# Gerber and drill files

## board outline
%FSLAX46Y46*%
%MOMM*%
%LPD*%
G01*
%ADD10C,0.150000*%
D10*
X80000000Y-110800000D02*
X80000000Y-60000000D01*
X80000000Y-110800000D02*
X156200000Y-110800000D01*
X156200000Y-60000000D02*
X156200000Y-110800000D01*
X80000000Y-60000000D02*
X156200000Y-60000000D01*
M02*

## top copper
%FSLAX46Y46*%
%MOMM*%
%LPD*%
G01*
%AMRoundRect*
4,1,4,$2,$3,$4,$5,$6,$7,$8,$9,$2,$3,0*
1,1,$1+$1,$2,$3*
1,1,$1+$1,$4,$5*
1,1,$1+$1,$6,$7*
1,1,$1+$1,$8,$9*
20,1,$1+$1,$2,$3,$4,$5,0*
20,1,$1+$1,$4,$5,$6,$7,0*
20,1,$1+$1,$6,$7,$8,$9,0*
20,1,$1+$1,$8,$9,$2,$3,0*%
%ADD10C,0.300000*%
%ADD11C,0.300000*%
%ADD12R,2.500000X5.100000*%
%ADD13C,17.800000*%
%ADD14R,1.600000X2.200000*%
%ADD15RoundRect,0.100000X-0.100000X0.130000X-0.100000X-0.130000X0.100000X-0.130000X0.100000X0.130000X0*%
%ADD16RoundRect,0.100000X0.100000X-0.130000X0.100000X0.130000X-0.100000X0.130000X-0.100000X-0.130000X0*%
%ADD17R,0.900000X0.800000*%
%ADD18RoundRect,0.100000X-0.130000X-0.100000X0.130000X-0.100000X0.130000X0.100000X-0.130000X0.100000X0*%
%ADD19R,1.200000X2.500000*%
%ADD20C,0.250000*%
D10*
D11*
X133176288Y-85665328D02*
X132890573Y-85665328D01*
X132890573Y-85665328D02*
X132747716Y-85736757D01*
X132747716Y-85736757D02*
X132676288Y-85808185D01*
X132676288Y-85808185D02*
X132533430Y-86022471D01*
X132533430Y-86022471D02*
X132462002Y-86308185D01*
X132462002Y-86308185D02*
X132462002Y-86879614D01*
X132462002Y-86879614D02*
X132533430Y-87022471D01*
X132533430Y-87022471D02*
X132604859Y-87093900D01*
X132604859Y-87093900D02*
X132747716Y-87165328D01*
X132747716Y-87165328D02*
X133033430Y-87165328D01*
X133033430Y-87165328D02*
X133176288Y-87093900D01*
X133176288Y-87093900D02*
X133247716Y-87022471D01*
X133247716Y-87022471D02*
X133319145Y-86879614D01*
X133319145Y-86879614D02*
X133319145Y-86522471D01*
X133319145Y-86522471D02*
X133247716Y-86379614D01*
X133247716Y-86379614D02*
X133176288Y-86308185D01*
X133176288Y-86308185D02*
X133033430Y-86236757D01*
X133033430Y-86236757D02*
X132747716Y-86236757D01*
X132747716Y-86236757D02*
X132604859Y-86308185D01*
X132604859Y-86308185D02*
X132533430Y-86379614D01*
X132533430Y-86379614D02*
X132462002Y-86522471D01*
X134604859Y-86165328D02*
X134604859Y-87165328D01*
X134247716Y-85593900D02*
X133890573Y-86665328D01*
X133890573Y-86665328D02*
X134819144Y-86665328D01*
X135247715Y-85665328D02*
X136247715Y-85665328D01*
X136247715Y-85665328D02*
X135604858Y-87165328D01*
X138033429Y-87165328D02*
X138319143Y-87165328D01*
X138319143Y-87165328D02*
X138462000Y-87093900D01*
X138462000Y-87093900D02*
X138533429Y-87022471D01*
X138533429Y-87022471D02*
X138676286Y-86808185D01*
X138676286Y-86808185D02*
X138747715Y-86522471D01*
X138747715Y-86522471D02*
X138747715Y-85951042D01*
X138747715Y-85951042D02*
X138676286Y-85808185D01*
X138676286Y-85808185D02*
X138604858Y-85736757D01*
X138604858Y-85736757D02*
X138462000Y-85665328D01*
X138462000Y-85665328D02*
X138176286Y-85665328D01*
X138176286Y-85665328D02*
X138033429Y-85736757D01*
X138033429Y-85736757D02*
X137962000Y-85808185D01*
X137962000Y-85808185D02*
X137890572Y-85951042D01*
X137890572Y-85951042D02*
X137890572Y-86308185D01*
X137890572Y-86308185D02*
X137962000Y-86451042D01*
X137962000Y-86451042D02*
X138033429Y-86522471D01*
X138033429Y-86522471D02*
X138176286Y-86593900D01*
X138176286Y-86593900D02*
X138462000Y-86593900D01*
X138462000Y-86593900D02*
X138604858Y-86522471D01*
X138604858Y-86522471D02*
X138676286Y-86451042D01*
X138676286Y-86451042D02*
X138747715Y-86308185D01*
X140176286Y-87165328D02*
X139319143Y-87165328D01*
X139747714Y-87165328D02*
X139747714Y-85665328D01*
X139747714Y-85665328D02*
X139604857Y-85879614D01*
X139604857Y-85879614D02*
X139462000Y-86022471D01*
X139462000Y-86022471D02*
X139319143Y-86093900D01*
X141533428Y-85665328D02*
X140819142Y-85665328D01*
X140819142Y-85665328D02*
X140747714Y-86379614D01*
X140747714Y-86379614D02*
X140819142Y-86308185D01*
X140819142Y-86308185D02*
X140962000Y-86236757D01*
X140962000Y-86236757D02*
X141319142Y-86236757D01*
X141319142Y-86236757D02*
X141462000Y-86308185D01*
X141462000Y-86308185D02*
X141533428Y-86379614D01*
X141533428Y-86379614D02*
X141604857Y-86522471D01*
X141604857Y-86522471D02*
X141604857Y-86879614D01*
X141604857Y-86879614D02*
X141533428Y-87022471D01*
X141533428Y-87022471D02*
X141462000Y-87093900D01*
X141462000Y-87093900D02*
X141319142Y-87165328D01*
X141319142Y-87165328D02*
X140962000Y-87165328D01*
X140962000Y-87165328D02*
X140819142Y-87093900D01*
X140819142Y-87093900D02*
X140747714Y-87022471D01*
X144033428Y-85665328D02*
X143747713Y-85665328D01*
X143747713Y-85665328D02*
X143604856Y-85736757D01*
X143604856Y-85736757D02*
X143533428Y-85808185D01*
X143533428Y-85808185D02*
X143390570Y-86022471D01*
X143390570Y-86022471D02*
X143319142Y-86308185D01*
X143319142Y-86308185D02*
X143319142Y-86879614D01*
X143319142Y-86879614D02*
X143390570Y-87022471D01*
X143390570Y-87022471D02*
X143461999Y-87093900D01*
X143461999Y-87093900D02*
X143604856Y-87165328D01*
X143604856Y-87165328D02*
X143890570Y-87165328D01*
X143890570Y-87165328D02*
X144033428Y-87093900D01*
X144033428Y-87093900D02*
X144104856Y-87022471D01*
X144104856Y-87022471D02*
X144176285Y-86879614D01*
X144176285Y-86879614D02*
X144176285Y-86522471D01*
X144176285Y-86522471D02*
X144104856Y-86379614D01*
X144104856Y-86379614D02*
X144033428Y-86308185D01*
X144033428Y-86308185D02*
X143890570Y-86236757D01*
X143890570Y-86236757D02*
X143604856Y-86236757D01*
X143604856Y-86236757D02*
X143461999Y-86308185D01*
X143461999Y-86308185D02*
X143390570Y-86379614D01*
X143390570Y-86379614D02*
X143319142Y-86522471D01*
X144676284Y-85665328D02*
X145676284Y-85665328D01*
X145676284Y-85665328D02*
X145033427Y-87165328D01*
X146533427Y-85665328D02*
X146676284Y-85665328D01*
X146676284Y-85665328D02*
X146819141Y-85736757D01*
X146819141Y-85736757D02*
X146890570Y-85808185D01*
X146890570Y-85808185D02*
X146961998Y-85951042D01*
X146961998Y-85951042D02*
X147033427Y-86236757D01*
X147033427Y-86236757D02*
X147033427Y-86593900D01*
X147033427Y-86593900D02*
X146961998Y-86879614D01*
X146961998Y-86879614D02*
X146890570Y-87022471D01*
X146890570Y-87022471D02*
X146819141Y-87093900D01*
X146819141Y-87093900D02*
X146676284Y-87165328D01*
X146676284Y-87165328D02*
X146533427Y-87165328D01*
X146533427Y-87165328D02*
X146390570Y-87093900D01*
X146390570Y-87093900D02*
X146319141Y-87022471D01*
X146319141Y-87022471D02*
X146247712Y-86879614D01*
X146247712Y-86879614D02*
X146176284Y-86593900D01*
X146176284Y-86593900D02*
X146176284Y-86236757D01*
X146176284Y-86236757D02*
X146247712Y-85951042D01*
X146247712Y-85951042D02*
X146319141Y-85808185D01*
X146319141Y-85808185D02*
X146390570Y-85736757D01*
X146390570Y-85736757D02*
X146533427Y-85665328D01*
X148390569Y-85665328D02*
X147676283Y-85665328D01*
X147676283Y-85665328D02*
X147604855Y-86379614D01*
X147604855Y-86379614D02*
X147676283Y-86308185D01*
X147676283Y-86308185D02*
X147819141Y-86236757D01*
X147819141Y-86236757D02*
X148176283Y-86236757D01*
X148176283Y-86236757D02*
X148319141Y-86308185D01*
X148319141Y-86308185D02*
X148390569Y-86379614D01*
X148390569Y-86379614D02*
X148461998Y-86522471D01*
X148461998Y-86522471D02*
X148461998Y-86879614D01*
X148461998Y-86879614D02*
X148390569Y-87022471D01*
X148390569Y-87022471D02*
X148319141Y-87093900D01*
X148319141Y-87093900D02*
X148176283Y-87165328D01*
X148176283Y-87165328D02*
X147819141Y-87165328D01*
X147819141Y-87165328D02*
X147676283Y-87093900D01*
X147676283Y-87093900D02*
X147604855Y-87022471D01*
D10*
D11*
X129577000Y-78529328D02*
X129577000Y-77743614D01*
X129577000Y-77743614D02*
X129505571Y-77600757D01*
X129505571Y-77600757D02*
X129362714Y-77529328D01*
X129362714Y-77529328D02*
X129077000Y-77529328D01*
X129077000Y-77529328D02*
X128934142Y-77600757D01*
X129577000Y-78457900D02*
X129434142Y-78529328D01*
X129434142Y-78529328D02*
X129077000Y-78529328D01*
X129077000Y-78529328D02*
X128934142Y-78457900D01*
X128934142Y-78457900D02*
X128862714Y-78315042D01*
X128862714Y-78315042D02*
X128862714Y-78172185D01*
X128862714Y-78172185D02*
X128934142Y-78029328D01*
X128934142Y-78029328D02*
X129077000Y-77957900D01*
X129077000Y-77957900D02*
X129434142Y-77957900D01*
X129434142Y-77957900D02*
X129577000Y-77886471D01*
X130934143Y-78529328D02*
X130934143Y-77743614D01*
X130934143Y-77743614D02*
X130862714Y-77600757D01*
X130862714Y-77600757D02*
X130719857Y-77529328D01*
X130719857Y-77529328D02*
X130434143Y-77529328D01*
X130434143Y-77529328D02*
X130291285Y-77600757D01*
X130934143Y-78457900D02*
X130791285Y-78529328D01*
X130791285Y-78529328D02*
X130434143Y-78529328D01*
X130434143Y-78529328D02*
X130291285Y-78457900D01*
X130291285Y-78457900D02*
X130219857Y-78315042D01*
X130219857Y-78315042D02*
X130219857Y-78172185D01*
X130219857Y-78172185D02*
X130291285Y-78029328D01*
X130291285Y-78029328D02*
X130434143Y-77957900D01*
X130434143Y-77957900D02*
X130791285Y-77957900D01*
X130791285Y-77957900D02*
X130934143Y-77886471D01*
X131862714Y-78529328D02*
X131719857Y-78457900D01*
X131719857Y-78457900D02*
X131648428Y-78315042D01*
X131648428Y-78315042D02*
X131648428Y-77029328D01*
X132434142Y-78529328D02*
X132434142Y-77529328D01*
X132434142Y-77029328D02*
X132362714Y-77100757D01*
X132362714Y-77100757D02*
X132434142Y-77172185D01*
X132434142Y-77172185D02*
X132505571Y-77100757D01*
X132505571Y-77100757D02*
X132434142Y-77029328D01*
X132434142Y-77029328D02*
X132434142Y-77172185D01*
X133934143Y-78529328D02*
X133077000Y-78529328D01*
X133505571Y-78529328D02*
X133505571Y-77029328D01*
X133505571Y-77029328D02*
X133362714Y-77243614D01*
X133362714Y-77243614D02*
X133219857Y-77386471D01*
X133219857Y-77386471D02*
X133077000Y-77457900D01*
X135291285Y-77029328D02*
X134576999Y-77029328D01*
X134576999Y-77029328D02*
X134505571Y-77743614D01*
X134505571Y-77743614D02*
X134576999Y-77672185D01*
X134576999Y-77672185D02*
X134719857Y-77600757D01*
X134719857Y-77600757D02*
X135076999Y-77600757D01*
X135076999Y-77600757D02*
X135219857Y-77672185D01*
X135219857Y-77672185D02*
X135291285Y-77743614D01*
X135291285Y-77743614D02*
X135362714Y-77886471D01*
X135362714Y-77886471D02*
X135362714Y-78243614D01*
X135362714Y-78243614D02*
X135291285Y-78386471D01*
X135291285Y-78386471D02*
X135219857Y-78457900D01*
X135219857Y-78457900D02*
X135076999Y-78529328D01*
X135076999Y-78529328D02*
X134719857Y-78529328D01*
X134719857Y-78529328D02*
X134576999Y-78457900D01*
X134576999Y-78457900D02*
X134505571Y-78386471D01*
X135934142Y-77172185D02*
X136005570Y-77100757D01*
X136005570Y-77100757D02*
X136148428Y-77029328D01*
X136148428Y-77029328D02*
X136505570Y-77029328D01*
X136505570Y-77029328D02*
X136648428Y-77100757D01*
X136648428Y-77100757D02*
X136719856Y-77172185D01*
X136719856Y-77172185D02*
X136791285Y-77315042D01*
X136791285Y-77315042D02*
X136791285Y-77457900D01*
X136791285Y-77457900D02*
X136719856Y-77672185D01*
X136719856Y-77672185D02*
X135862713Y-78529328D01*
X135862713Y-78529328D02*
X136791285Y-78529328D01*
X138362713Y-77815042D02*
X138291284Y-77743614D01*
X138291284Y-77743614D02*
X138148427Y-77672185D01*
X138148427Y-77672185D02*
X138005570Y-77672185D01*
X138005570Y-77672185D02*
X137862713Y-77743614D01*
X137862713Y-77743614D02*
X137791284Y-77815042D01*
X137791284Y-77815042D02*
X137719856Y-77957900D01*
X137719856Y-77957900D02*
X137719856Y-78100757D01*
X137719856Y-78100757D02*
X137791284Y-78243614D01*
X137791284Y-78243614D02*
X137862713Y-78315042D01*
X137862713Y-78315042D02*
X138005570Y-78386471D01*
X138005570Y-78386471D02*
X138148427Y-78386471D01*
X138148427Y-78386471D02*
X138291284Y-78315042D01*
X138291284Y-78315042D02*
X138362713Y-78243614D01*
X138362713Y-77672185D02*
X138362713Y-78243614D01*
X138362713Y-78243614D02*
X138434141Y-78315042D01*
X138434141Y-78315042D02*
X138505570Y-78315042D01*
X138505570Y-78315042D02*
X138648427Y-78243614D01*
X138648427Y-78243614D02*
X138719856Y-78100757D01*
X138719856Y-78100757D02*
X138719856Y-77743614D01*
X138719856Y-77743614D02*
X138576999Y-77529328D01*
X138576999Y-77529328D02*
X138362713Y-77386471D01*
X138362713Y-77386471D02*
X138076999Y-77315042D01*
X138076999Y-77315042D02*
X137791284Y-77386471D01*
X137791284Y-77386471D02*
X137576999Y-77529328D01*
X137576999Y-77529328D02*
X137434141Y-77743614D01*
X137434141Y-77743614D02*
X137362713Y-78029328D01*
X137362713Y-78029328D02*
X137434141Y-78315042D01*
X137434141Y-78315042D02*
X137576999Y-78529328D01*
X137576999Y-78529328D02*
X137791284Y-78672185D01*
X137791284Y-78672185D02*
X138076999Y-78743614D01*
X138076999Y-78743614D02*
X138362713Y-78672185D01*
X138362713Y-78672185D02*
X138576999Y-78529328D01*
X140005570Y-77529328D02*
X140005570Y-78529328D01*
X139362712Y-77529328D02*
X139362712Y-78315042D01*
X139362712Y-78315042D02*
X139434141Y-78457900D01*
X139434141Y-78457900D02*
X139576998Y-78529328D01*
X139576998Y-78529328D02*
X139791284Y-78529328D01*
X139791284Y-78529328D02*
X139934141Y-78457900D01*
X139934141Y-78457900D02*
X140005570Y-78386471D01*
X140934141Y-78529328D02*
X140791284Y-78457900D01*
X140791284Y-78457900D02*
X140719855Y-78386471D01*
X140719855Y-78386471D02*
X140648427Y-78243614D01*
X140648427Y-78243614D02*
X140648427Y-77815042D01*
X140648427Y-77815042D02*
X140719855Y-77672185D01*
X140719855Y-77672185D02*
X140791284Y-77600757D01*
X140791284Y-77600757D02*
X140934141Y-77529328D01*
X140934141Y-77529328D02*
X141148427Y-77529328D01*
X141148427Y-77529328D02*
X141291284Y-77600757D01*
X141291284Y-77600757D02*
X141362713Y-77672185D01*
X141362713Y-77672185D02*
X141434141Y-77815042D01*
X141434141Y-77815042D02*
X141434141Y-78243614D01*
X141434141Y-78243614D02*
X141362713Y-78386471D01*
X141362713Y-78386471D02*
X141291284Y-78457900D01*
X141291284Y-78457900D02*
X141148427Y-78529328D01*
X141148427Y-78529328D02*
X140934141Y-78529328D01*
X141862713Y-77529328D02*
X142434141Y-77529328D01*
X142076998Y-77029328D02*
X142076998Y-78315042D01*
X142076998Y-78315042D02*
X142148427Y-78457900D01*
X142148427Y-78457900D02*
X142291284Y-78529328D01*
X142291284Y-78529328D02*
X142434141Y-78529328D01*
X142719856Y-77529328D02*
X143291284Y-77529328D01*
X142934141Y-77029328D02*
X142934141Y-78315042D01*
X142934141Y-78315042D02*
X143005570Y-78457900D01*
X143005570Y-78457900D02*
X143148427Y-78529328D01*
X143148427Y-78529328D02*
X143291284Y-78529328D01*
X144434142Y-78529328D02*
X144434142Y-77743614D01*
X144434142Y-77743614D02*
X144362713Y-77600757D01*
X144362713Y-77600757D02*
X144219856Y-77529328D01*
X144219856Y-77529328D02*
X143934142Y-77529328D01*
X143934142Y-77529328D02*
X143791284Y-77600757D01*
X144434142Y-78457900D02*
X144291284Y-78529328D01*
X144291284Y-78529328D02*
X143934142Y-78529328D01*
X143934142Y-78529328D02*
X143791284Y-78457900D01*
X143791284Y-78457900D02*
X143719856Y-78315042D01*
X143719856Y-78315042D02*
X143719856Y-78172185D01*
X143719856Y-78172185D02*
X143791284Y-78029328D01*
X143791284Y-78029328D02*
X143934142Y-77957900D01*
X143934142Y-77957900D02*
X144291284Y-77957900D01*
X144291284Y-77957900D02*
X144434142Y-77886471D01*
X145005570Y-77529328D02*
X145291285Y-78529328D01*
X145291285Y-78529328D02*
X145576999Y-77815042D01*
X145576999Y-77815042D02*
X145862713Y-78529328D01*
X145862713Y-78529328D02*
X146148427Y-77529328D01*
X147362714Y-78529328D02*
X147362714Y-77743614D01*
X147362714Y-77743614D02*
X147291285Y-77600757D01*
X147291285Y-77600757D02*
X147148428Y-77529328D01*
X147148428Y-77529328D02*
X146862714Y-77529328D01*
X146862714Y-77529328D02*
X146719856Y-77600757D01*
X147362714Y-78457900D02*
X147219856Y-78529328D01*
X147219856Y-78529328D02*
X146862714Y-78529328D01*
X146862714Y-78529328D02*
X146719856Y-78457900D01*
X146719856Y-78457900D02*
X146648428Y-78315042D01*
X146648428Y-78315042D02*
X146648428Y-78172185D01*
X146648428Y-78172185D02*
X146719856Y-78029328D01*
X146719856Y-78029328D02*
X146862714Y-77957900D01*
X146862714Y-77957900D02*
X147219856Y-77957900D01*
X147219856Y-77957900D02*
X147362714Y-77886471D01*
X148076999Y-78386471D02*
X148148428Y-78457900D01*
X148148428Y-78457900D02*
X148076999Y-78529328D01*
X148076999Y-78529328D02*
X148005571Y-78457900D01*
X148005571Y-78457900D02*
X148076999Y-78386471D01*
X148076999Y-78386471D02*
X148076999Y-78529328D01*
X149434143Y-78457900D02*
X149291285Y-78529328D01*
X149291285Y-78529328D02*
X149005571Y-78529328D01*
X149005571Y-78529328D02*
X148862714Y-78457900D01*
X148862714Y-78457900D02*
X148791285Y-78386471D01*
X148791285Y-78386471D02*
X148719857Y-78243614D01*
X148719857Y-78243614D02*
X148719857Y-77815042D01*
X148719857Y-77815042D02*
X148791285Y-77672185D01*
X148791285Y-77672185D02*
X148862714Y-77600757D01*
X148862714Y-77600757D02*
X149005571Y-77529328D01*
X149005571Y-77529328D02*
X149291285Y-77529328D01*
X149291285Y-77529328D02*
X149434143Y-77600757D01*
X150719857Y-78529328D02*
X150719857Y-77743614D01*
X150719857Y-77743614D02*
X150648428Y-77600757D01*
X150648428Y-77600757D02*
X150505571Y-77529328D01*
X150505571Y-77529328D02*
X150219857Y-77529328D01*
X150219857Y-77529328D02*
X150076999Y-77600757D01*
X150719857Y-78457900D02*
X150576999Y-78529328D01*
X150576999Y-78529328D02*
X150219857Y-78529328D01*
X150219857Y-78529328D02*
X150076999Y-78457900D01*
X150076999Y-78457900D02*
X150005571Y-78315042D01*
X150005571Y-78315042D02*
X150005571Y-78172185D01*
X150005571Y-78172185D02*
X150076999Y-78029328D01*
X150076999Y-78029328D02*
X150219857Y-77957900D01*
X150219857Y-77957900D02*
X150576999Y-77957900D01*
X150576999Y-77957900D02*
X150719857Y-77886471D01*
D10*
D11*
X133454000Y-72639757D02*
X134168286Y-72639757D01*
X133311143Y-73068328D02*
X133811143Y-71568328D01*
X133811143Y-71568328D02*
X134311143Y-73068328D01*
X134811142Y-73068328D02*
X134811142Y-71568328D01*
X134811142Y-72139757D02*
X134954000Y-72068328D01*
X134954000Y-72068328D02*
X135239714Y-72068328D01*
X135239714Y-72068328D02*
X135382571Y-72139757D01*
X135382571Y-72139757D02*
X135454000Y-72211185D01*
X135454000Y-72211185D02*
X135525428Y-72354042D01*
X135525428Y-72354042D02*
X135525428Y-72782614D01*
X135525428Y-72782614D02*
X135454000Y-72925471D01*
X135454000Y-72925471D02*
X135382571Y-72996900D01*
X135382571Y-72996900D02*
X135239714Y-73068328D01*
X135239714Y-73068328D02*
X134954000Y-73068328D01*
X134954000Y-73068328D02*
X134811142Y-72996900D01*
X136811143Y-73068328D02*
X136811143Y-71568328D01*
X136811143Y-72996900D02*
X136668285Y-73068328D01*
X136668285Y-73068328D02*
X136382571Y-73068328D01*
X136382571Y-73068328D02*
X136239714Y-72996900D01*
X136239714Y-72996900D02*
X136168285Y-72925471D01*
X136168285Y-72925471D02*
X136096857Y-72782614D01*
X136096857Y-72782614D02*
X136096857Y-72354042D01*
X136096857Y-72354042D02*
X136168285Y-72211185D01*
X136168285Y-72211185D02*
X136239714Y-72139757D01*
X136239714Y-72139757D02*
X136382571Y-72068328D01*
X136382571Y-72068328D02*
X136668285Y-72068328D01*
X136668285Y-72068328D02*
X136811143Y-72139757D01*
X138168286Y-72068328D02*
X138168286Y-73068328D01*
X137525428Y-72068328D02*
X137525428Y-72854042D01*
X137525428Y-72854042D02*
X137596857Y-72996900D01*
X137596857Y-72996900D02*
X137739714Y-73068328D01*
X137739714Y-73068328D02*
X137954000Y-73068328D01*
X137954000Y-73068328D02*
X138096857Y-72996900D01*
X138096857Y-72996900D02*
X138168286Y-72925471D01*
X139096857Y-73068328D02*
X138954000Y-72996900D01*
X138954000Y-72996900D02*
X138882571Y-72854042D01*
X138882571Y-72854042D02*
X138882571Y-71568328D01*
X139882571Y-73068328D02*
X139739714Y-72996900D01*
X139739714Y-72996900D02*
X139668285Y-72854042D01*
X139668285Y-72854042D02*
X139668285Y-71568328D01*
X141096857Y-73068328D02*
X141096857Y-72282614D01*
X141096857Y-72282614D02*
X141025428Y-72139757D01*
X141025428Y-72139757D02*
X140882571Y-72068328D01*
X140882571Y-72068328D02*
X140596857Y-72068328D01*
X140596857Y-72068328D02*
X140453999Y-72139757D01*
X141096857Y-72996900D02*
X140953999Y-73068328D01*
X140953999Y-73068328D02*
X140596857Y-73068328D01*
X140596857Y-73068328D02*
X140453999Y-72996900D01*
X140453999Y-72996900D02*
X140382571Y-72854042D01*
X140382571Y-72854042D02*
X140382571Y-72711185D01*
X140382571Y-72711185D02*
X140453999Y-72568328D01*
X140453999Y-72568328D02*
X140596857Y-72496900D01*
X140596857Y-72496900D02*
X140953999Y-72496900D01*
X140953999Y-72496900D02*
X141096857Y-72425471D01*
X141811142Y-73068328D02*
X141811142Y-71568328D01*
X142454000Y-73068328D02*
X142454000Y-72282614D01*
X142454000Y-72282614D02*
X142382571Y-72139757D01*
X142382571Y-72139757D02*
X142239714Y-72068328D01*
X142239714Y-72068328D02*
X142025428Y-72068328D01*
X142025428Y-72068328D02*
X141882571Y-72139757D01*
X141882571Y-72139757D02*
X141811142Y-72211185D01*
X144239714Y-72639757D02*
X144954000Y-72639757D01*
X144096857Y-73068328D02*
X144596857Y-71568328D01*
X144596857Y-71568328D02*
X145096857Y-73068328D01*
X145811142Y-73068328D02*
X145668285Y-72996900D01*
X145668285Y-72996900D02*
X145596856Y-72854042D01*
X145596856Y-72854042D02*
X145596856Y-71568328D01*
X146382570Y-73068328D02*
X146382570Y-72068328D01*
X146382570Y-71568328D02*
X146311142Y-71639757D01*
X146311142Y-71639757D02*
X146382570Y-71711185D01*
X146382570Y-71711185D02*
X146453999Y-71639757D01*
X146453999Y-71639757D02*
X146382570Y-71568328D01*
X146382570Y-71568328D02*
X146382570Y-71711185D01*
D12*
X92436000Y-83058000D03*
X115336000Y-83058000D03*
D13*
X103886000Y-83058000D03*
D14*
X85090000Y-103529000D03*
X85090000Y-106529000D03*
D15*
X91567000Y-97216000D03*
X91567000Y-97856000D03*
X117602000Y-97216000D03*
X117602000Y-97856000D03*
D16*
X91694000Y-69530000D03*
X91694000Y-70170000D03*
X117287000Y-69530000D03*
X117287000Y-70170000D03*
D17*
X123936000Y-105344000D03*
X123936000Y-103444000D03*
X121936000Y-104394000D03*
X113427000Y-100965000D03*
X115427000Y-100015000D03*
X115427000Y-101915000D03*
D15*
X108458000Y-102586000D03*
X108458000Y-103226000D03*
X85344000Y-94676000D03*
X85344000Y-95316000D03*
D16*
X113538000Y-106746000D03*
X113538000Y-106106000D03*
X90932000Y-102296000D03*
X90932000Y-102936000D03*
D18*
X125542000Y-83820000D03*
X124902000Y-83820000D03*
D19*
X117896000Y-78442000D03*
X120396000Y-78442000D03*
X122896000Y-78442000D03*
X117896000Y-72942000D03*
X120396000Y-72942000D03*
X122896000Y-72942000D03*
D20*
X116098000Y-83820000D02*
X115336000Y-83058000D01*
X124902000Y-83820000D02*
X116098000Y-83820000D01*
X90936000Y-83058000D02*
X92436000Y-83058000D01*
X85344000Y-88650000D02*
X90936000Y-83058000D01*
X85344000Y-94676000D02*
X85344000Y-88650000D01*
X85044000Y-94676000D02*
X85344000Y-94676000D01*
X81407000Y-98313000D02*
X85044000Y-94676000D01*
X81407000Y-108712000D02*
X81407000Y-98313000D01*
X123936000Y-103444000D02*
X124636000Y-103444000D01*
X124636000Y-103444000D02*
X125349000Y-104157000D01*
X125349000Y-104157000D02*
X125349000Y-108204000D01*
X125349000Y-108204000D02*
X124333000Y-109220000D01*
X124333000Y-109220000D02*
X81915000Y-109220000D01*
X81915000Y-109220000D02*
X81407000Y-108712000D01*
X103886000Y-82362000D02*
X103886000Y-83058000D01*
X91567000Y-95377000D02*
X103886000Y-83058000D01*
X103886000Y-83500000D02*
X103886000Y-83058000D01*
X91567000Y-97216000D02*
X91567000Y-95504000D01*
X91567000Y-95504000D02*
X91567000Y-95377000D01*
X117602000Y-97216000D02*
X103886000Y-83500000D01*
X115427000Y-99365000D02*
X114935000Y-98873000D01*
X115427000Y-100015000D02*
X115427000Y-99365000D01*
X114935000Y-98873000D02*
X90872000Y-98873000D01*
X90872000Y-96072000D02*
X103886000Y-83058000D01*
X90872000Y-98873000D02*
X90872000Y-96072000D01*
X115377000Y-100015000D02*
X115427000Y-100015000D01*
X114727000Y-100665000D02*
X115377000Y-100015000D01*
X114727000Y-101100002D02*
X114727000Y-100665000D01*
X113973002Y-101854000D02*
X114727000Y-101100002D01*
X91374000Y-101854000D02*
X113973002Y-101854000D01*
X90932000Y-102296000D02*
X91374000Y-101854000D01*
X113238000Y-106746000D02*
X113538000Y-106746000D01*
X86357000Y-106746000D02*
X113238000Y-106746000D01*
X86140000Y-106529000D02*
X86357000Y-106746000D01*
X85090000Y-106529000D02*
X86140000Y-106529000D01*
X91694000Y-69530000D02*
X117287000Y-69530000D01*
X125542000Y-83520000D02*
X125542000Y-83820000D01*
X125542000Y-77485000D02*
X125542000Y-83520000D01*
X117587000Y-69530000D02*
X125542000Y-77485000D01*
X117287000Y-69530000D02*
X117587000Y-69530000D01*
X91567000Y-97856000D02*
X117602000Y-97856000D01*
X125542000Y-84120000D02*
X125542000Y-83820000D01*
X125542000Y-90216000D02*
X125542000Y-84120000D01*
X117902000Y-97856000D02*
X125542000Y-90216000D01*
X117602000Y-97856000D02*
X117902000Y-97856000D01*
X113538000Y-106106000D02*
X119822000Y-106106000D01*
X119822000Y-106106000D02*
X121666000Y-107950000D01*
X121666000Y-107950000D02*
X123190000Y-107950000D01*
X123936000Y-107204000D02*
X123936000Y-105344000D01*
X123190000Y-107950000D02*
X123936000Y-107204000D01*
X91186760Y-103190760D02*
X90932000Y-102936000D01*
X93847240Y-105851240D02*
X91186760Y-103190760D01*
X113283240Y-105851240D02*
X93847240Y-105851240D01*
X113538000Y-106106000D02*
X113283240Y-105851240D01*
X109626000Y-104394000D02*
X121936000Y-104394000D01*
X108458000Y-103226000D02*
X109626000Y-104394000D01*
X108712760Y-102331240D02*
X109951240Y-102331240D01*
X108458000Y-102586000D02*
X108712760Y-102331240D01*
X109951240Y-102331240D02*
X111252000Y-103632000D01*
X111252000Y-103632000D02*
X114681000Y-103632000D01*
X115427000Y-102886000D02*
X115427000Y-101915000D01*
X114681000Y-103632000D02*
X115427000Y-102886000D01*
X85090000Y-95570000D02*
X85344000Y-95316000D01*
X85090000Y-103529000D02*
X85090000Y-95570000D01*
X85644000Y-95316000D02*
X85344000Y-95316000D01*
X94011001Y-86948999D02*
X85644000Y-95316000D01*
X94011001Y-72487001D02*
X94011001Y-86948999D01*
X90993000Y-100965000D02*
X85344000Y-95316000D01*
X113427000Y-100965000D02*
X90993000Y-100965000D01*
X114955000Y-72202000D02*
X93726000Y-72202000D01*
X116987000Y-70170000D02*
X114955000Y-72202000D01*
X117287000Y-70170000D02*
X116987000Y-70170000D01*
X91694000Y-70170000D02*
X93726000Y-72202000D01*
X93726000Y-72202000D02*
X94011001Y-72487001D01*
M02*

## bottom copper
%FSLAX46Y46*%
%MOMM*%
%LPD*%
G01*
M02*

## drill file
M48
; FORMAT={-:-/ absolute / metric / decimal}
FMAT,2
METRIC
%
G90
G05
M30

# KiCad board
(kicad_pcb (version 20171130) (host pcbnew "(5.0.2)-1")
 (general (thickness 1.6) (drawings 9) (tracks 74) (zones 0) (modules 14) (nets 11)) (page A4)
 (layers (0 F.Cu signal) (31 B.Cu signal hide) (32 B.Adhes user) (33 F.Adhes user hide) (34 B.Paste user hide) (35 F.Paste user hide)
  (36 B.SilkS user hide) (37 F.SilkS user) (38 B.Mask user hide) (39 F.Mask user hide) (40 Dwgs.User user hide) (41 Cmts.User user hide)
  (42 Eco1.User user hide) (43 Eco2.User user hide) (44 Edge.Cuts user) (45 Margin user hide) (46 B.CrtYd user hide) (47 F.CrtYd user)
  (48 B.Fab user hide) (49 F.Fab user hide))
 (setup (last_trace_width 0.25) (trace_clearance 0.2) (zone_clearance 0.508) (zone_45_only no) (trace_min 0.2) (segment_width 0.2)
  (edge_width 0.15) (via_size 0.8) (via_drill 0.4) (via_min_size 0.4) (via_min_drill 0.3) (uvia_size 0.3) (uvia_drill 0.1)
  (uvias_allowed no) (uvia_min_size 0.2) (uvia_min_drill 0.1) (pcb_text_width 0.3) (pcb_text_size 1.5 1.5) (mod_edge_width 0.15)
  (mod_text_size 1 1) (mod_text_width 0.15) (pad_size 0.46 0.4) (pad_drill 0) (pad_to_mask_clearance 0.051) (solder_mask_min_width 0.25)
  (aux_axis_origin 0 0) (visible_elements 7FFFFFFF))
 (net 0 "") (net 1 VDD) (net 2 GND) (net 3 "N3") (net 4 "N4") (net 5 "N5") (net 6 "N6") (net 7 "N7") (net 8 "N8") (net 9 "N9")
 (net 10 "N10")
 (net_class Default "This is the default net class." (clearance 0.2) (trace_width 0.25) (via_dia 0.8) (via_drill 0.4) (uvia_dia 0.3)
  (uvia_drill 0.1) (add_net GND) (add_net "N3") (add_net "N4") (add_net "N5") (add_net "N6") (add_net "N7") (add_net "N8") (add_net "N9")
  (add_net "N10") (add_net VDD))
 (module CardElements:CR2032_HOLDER (layer F.Cu) (at 103.886 83.058)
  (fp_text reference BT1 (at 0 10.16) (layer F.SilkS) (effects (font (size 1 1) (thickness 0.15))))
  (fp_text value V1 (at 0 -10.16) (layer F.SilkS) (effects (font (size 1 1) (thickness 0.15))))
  (pad 1 smd rect (at -11.45 0) (size 2.5 5.1) (layers F.Cu F.Paste F.Mask) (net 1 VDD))
  (pad 1 smd rect (at 11.45 0) (size 2.5 5.1) (layers F.Cu F.Paste F.Mask) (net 1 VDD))
  (pad 2 smd circle (at 0 0) (size 17.8 17.8) (layers F.Cu F.Paste F.Mask) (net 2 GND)))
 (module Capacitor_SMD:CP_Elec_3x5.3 (layer F.Cu) (at 85.09 105.029 270)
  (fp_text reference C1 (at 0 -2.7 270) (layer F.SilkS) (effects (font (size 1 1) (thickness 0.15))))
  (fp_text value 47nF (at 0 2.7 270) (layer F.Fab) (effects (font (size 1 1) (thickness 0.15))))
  (pad 1 smd rect (at -1.5 0 270) (size 2.2 1.6) (layers F.Cu F.Paste F.Mask) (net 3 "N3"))
  (pad 2 smd rect (at 1.5 0 270) (size 2.2 1.6) (layers F.Cu F.Paste F.Mask) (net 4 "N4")))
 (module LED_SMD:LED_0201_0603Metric (layer F.Cu) (at 91.567 97.536 270)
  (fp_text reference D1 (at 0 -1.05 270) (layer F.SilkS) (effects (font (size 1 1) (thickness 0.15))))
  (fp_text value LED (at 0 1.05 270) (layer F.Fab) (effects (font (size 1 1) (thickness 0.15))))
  (pad "" smd roundrect (at -0.345 0 270) (size 0.318 0.36) (layers F.Paste) (roundrect_rratio 0.25))
  (pad "" smd roundrect (at 0.345 0 270) (size 0.318 0.36) (layers F.Paste) (roundrect_rratio 0.25))
  (pad 1 smd roundrect (at -0.32 0 270) (size 0.46 0.4) (layers F.Cu F.Mask) (roundrect_rratio 0.25) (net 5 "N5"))
  (pad 2 smd roundrect (at 0.32 0 270) (size 0.46 0.4) (layers F.Cu F.Mask) (roundrect_rratio 0.25) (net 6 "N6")))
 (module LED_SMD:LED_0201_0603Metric (layer F.Cu) (at 117.602 97.536 270)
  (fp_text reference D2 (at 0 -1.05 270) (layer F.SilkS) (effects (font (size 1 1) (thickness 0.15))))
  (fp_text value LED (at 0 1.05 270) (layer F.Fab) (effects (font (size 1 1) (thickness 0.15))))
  (pad "" smd roundrect (at -0.345 0 270) (size 0.318 0.36) (layers F.Paste) (roundrect_rratio 0.25))
  (pad "" smd roundrect (at 0.345 0 270) (size 0.318 0.36) (layers F.Paste) (roundrect_rratio 0.25))
  (pad 1 smd roundrect (at -0.32 0 270) (size 0.46 0.4) (layers F.Cu F.Mask) (roundrect_rratio 0.25) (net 5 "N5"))
  (pad 2 smd roundrect (at 0.32 0 270) (size 0.46 0.4) (layers F.Cu F.Mask) (roundrect_rratio 0.25) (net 6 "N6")))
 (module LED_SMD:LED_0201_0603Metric (layer F.Cu) (at 91.694 69.85 90)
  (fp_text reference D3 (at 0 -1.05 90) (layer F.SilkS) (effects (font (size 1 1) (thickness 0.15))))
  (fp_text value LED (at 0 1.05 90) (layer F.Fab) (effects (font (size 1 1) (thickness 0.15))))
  (pad 2 smd roundrect (at 0.32 0 90) (size 0.46 0.4) (layers F.Cu F.Mask) (roundrect_rratio 0.25) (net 6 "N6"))
  (pad 1 smd roundrect (at -0.32 0 90) (size 0.46 0.4) (layers F.Cu F.Mask) (roundrect_rratio 0.25) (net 5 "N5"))
  (pad "" smd roundrect (at 0.345 0 90) (size 0.318 0.36) (layers F.Paste) (roundrect_rratio 0.25))
  (pad "" smd roundrect (at -0.345 0 90) (size 0.318 0.36) (layers F.Paste) (roundrect_rratio 0.25)))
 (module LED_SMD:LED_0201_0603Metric (layer F.Cu) (at 117.287 69.85 90)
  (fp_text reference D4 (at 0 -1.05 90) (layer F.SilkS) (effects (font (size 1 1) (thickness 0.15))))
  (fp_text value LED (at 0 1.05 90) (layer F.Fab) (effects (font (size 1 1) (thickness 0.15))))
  (pad 2 smd roundrect (at 0.32 0 90) (size 0.46 0.4) (layers F.Cu F.Mask) (roundrect_rratio 0.25) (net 6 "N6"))
  (pad 1 smd roundrect (at -0.32 0 90) (size 0.46 0.4) (layers F.Cu F.Mask) (roundrect_rratio 0.25) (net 5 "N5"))
  (pad "" smd roundrect (at 0.345 0 90) (size 0.318 0.36) (layers F.Paste) (roundrect_rratio 0.25))
  (pad "" smd roundrect (at -0.345 0 90) (size 0.318 0.36) (layers F.Paste) (roundrect_rratio 0.25)))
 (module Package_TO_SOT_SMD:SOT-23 (layer F.Cu) (at 122.936 104.394 180)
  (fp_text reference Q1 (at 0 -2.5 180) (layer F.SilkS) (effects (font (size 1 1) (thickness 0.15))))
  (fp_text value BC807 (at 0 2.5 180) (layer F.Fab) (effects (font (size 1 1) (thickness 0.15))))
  (pad 1 smd rect (at -1 -0.95 180) (size 0.9 0.8) (layers F.Cu F.Paste F.Mask) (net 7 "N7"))
  (pad 2 smd rect (at -1 0.95 180) (size 0.9 0.8) (layers F.Cu F.Paste F.Mask) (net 1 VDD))
  (pad 3 smd rect (at 1 0 180) (size 0.9 0.8) (layers F.Cu F.Paste F.Mask) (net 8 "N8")))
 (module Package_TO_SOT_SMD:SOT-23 (layer F.Cu) (at 114.427 100.965 180)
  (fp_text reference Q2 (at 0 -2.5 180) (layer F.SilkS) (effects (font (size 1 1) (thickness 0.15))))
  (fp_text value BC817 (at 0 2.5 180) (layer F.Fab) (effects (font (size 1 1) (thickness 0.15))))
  (pad 3 smd rect (at 1 0 180) (size 0.9 0.8) (layers F.Cu F.Paste F.Mask) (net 3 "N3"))
  (pad 2 smd rect (at -1 0.95 180) (size 0.9 0.8) (layers F.Cu F.Paste F.Mask) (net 2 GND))
  (pad 1 smd rect (at -1 -0.95 180) (size 0.9 0.8) (layers F.Cu F.Paste F.Mask) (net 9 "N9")))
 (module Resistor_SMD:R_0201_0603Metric (layer F.Cu) (at 108.458 102.906 270)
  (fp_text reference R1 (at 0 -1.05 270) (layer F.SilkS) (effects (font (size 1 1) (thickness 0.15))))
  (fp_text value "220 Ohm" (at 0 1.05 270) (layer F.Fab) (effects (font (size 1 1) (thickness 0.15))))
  (pad "" smd roundrect (at -0.345 0 270) (size 0.318 0.36) (layers F.Paste) (roundrect_rratio 0.25))
  (pad "" smd roundrect (at 0.345 0 270) (size 0.318 0.36) (layers F.Paste) (roundrect_rratio 0.25))
  (pad 1 smd roundrect (at -0.32 0 270) (size 0.46 0.4) (layers F.Cu F.Mask) (roundrect_rratio 0.25) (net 9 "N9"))
  (pad 2 smd roundrect (at 0.32 0 270) (size 0.46 0.4) (layers F.Cu F.Mask) (roundrect_rratio 0.25) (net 8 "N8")))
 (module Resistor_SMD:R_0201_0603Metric (layer F.Cu) (at 85.344 94.996 270)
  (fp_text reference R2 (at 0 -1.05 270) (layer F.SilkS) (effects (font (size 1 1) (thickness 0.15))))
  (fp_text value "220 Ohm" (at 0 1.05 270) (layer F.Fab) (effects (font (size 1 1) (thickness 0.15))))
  (pad "" smd roundrect (at -0.345 0 270) (size 0.318 0.36) (layers F.Paste) (roundrect_rratio 0.25))
  (pad "" smd roundrect (at 0.345 0 270) (size 0.318 0.36) (layers F.Paste) (roundrect_rratio 0.25))
  (pad 1 smd roundrect (at -0.32 0 270) (size 0.46 0.4) (layers F.Cu F.Mask) (roundrect_rratio 0.25) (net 1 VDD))
  (pad 2 smd roundrect (at 0.32 0 270) (size 0.46 0.4) (layers F.Cu F.Mask) (roundrect_rratio 0.25) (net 3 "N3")))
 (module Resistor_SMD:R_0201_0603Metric (layer F.Cu) (at 113.538 106.426 90)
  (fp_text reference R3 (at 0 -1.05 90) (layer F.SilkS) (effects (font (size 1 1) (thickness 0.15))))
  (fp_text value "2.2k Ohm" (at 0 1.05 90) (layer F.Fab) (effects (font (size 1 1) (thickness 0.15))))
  (pad "" smd roundrect (at -0.345 0 90) (size 0.318 0.36) (layers F.Paste) (roundrect_rratio 0.25))
  (pad "" smd roundrect (at 0.345 0 90) (size 0.318 0.36) (layers F.Paste) (roundrect_rratio 0.25))
  (pad 1 smd roundrect (at -0.32 0 90) (size 0.46 0.4) (layers F.Cu F.Mask) (roundrect_rratio 0.25) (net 4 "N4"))
  (pad 2 smd roundrect (at 0.32 0 90) (size 0.46 0.4) (layers F.Cu F.Mask) (roundrect_rratio 0.25) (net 7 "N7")))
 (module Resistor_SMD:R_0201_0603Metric (layer F.Cu) (at 90.932 102.616 90)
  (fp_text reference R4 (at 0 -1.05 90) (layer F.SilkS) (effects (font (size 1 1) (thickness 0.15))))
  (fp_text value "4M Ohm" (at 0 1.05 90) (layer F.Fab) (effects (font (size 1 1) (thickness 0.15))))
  (pad 2 smd roundrect (at 0.32 0 90) (size 0.46 0.4) (layers F.Cu F.Mask) (roundrect_rratio 0.25) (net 2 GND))
  (pad 1 smd roundrect (at -0.32 0 90) (size 0.46 0.4) (layers F.Cu F.Mask) (roundrect_rratio 0.25) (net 7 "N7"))
  (pad "" smd roundrect (at 0.345 0 90) (size 0.318 0.36) (layers F.Paste) (roundrect_rratio 0.25))
  (pad "" smd roundrect (at -0.345 0 90) (size 0.318 0.36) (layers F.Paste) (roundrect_rratio 0.25)))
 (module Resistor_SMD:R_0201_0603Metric (layer F.Cu) (at 125.222 83.82)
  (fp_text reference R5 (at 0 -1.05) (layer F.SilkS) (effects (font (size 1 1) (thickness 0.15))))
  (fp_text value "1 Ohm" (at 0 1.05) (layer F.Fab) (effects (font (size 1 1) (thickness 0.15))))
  (pad 2 smd roundrect (at 0.32 0) (size 0.46 0.4) (layers F.Cu F.Mask) (roundrect_rratio 0.25) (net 6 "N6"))
  (pad 1 smd roundrect (at -0.32 0) (size 0.46 0.4) (layers F.Cu F.Mask) (roundrect_rratio 0.25) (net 1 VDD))
  (pad "" smd roundrect (at 0.345 0) (size 0.318 0.36) (layers F.Paste) (roundrect_rratio 0.25))
  (pad "" smd roundrect (at -0.345 0) (size 0.318 0.36) (layers F.Paste) (roundrect_rratio 0.25)))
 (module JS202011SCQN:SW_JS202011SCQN (layer F.Cu) (at 120.396 75.692)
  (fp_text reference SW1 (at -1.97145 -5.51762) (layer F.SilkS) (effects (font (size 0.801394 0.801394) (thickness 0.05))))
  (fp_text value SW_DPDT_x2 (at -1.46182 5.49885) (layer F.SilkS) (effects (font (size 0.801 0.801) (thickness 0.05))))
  (pad 1 smd rect (at -2.5 2.75) (size 1.2 2.5) (layers F.Cu F.Paste F.Mask) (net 5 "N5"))
  (pad 2 smd rect (at 0 2.75) (size 1.2 2.5) (layers F.Cu F.Paste F.Mask) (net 3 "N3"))
  (pad 3 smd rect (at 2.5 2.75) (size 1.2 2.5) (layers F.Cu F.Paste F.Mask) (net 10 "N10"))
  (pad 4 smd rect (at -2.5 -2.75) (size 1.2 2.5) (layers F.Cu F.Paste F.Mask))
  (pad 5 smd rect (at 0 -2.75) (size 1.2 2.5) (layers F.Cu F.Paste F.Mask))
  (pad 6 smd rect (at 2.5 -2.75) (size 1.2 2.5) (layers F.Cu F.Paste F.Mask)))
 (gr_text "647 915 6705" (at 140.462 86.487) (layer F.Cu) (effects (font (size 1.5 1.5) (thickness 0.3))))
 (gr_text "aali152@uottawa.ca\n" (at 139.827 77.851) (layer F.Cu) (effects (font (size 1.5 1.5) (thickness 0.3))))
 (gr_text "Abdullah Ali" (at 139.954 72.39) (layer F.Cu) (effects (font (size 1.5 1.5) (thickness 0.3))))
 (gr_line (start 80 110.8) (end 80 60) (layer Edge.Cuts) (width 0.15))
 (gr_line (start 80 110.8) (end 156.2 110.8) (layer Edge.Cuts) (width 0.15))
 (gr_line (start 156.2 60) (end 156.2 110.8) (layer Edge.Cuts) (width 0.15))
 (gr_line (start 80 60) (end 156.2 60) (layer Edge.Cuts) (width 0.15))
 (segment (start 116.098 83.82) (end 115.336 83.058) (width 0.25) (layer F.Cu) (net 1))
 (segment (start 124.902 83.82) (end 116.098 83.82) (width 0.25) (layer F.Cu) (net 1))
 (segment (start 90.936 83.058) (end 92.436 83.058) (width 0.25) (layer F.Cu) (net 1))
 (segment (start 85.344 88.65) (end 90.936 83.058) (width 0.25) (layer F.Cu) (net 1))
 (segment (start 85.344 94.676) (end 85.344 88.65) (width 0.25) (layer F.Cu) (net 1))
 (segment (start 85.044 94.676) (end 85.344 94.676) (width 0.25) (layer F.Cu) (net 1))
 (segment (start 81.407 98.313) (end 85.044 94.676) (width 0.25) (layer F.Cu) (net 1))
 (segment (start 81.407 108.712) (end 81.407 98.313) (width 0.25) (layer F.Cu) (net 1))
 (segment (start 123.936 103.444) (end 124.636 103.444) (width 0.25) (layer F.Cu) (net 1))
 (segment (start 124.636 103.444) (end 125.349 104.157) (width 0.25) (layer F.Cu) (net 1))
 (segment (start 125.349 104.157) (end 125.349 108.204) (width 0.25) (layer F.Cu) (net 1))
 (segment (start 125.349 108.204) (end 124.333 109.22) (width 0.25) (layer F.Cu) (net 1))
 (segment (start 124.333 109.22) (end 81.915 109.22) (width 0.25) (layer F.Cu) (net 1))
 (segment (start 81.915 109.22) (end 81.407 108.712) (width 0.25) (layer F.Cu) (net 1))
 (segment (start 103.886 82.362) (end 103.886 83.058) (width 0.25) (layer F.Cu) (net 2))
 (segment (start 91.567 95.377) (end 103.886 83.058) (width 0.25) (layer F.Cu) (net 2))
 (segment (start 103.886 83.5) (end 103.886 83.058) (width 0.25) (layer F.Cu) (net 2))
 (segment (start 91.567 97.216) (end 91.567 95.504) (width 0.25) (layer F.Cu) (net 2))
 (segment (start 91.567 95.504) (end 91.567 95.377) (width 0.25) (layer F.Cu) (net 2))
 (segment (start 117.602 97.216) (end 103.886 83.5) (width 0.25) (layer F.Cu) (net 2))
 (segment (start 115.427 99.365) (end 114.935 98.873) (width 0.25) (layer F.Cu) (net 2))
 (segment (start 115.427 100.015) (end 115.427 99.365) (width 0.25) (layer F.Cu) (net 2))
 (segment (start 114.935 98.873) (end 90.872 98.873) (width 0.25) (layer F.Cu) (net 2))
 (segment (start 90.872 96.072) (end 103.886 83.058) (width 0.25) (layer F.Cu) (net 2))
 (segment (start 90.872 98.873) (end 90.872 96.072) (width 0.25) (layer F.Cu) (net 2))
 (segment (start 115.377 100.015) (end 115.427 100.015) (width 0.25) (layer F.Cu) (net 2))
 (segment (start 114.727 100.665) (end 115.377 100.015) (width 0.25) (layer F.Cu) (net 2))
 (segment (start 114.727 101.100002) (end 114.727 100.665) (width 0.25) (layer F.Cu) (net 2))
 (segment (start 113.973002 101.854) (end 114.727 101.100002) (width 0.25) (layer F.Cu) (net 2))
 (segment (start 91.374 101.854) (end 113.973002 101.854) (width 0.25) (layer F.Cu) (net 2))
 (segment (start 90.932 102.296) (end 91.374 101.854) (width 0.25) (layer F.Cu) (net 2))
 (segment (start 113.238 106.746) (end 113.538 106.746) (width 0.25) (layer F.Cu) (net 4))
 (segment (start 86.357 106.746) (end 113.238 106.746) (width 0.25) (layer F.Cu) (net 4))
 (segment (start 86.14 106.529) (end 86.357 106.746) (width 0.25) (layer F.Cu) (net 4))
 (segment (start 85.09 106.529) (end 86.14 106.529) (width 0.25) (layer F.Cu) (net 4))
 (segment (start 91.694 69.53) (end 117.287 69.53) (width 0.25) (layer F.Cu) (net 6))
 (segment (start 125.542 83.52) (end 125.542 83.82) (width 0.25) (layer F.Cu) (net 6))
 (segment (start 125.542 77.485) (end 125.542 83.52) (width 0.25) (layer F.Cu) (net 6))
 (segment (start 117.587 69.53) (end 125.542 77.485) (width 0.25) (layer F.Cu) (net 6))
 (segment (start 117.287 69.53) (end 117.587 69.53) (width 0.25) (layer F.Cu) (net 6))
 (segment (start 91.567 97.856) (end 117.602 97.856) (width 0.25) (layer F.Cu) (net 6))
 (segment (start 125.542 84.12) (end 125.542 83.82) (width 0.25) (layer F.Cu) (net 6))
 (segment (start 125.542 90.216) (end 125.542 84.12) (width 0.25) (layer F.Cu) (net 6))
 (segment (start 117.902 97.856) (end 125.542 90.216) (width 0.25) (layer F.Cu) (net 6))
 (segment (start 117.602 97.856) (end 117.902 97.856) (width 0.25) (layer F.Cu) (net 6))
 (segment (start 113.538 106.106) (end 119.822 106.106) (width 0.25) (layer F.Cu) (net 7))
 (segment (start 119.822 106.106) (end 121.666 107.95) (width 0.25) (layer F.Cu) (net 7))
 (segment (start 121.666 107.95) (end 123.19 107.95) (width 0.25) (layer F.Cu) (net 7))
 (segment (start 123.936 107.204) (end 123.936 105.344) (width 0.25) (layer F.Cu) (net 7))
 (segment (start 123.19 107.95) (end 123.936 107.204) (width 0.25) (layer F.Cu) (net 7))
 (segment (start 91.18676 103.19076) (end 90.932 102.936) (width 0.25) (layer F.Cu) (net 7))
 (segment (start 93.84724 105.85124) (end 91.18676 103.19076) (width 0.25) (layer F.Cu) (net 7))
 (segment (start 113.28324 105.85124) (end 93.84724 105.85124) (width 0.25) (layer F.Cu) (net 7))
 (segment (start 113.538 106.106) (end 113.28324 105.85124) (width 0.25) (layer F.Cu) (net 7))
 (segment (start 109.626 104.394) (end 121.936 104.394) (width 0.25) (layer F.Cu) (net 8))
 (segment (start 108.458 103.226) (end 109.626 104.394) (width 0.25) (layer F.Cu) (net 8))
 (segment (start 108.71276 102.33124) (end 109.95124 102.33124) (width 0.25) (layer F.Cu) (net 9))
 (segment (start 108.458 102.586) (end 108.71276 102.33124) (width 0.25) (layer F.Cu) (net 9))
 (segment (start 109.95124 102.33124) (end 111.252 103.632) (width 0.25) (layer F.Cu) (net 9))
 (segment (start 111.252 103.632) (end 114.681 103.632) (width 0.25) (layer F.Cu) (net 9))
 (segment (start 115.427 102.886) (end 115.427 101.915) (width 0.25) (layer F.Cu) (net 9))
 (segment (start 114.681 103.632) (end 115.427 102.886) (width 0.25) (layer F.Cu) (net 9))
 (segment (start 85.09 95.57) (end 85.344 95.316) (width 0.25) (layer F.Cu) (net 3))
 (segment (start 85.09 103.529) (end 85.09 95.57) (width 0.25) (layer F.Cu) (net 3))
 (segment (start 85.644 95.316) (end 85.344 95.316) (width 0.25) (layer F.Cu) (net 3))
 (segment (start 94.011001 86.948999) (end 85.644 95.316) (width 0.25) (layer F.Cu) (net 3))
 (segment (start 94.011001 72.487001) (end 94.011001 86.948999) (width 0.25) (layer F.Cu) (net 3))
 (segment (start 90.993 100.965) (end 85.344 95.316) (width 0.25) (layer F.Cu) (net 3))
 (segment (start 113.427 100.965) (end 90.993 100.965) (width 0.25) (layer F.Cu) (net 3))
 (segment (start 114.955 72.202) (end 93.726 72.202) (width 0.25) (layer F.Cu) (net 3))
 (segment (start 116.987 70.17) (end 114.955 72.202) (width 0.25) (layer F.Cu) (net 3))
 (segment (start 117.287 70.17) (end 116.987 70.17) (width 0.25) (layer F.Cu) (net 3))
 (segment (start 91.694 70.17) (end 93.726 72.202) (width 0.25) (layer F.Cu) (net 3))
 (segment (start 93.726 72.202) (end 94.011001 72.487001) (width 0.25) (layer F.Cu) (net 3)))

